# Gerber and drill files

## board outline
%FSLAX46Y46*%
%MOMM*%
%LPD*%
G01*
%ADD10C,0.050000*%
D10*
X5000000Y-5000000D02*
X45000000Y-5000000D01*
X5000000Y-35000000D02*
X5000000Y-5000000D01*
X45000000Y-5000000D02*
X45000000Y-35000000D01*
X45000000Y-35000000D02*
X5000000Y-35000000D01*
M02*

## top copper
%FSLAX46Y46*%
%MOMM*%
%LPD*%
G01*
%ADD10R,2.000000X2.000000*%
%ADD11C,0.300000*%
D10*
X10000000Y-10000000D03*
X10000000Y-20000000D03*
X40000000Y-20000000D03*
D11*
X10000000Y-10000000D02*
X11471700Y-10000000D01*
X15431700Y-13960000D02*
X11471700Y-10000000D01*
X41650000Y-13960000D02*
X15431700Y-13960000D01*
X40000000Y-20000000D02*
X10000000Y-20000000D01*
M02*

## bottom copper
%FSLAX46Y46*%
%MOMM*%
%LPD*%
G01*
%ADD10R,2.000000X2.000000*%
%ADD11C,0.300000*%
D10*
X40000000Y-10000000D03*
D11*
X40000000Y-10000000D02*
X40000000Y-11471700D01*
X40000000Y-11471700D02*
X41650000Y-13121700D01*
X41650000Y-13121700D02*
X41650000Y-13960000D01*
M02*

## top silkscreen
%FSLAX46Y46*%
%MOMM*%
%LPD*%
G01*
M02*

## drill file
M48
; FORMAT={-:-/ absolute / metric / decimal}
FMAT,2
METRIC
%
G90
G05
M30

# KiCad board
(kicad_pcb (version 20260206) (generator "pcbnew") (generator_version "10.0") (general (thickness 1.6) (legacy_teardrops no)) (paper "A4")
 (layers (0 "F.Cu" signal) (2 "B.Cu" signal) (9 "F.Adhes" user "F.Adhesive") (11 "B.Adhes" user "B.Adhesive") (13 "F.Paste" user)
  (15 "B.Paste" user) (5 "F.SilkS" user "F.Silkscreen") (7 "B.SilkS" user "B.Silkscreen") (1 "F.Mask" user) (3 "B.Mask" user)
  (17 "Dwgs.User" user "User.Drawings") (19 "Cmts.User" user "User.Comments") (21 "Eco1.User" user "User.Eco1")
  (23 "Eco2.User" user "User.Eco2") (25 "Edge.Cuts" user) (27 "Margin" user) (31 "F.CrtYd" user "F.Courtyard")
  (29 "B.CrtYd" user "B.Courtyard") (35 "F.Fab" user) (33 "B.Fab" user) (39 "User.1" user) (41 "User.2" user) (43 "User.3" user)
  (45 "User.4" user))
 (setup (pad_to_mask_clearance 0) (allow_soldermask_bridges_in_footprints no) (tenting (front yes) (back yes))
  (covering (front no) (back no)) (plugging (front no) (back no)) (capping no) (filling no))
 (gr_line (start 5 5) (end 45 5) (stroke (width 0.05) (type default)) (layer "Edge.Cuts"))
 (gr_line (start 5 35) (end 5 5) (stroke (width 0.05) (type default)) (layer "Edge.Cuts"))
 (gr_line (start 45 5) (end 45 35) (stroke (width 0.05) (type default)) (layer "Edge.Cuts"))
 (gr_line (start 45 35) (end 5 35) (stroke (width 0.05) (type default)) (layer "Edge.Cuts"))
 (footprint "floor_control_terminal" (layer "F.Cu") (at 10 10)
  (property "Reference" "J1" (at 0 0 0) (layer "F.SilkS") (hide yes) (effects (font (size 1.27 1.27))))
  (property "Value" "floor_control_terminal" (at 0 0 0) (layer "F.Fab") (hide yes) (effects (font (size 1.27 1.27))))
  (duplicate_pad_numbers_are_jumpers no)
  (pad "1" smd rect (at 0 0) (size 2 2) (layers "F.Cu" "F.Paste" "F.Mask") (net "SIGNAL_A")))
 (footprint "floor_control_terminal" (layer "B.Cu") (at 40 10)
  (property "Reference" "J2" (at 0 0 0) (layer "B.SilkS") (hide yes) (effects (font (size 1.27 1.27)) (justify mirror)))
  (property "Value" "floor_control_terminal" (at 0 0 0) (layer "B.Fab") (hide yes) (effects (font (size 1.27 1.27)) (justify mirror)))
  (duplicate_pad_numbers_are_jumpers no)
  (pad "1" smd rect (at 0 0) (size 2 2) (layers "B.Cu" "B.Paste" "B.Mask") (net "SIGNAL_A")))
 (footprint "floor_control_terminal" (layer "F.Cu") (at 10 20)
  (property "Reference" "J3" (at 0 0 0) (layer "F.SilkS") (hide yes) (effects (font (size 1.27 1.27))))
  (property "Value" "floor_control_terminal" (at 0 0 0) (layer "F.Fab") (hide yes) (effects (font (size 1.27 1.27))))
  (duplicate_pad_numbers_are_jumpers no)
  (pad "1" smd rect (at 0 0) (size 2 2) (layers "F.Cu" "F.Paste" "F.Mask") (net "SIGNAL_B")))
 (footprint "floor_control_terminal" (layer "F.Cu") (at 40 20)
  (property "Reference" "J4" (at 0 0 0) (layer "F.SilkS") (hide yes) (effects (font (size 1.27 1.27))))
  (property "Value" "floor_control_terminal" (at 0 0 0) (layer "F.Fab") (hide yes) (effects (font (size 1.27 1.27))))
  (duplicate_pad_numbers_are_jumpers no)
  (pad "1" smd rect (at 0 0) (size 2 2) (layers "F.Cu" "F.Paste" "F.Mask") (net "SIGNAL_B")))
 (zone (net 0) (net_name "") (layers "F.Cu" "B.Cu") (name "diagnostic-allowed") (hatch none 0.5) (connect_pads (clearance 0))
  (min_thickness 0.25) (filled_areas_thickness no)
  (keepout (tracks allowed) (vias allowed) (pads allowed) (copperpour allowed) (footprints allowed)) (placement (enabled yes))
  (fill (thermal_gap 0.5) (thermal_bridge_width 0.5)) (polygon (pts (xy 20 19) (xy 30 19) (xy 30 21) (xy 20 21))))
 (segment (start 10 10) (end 11.4717 10) (width 0.3) (layer "F.Cu") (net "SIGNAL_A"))
 (segment (start 15.4317 13.96) (end 11.4717 10) (width 0.3) (layer "F.Cu") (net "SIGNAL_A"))
 (segment (start 41.65 13.96) (end 15.4317 13.96) (width 0.3) (layer "F.Cu") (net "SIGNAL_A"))
 (segment (start 40 10) (end 40 11.4717) (width 0.3) (layer "B.Cu") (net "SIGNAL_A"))
 (segment (start 40 11.4717) (end 41.65 13.1217) (width 0.3) (layer "B.Cu") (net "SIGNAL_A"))
 (segment (start 41.65 13.1217) (end 41.65 13.96) (width 0.3) (layer "B.Cu") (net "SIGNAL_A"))
 (segment (start 40 20) (end 10 20) (width 0.3) (layer "F.Cu") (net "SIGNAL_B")))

